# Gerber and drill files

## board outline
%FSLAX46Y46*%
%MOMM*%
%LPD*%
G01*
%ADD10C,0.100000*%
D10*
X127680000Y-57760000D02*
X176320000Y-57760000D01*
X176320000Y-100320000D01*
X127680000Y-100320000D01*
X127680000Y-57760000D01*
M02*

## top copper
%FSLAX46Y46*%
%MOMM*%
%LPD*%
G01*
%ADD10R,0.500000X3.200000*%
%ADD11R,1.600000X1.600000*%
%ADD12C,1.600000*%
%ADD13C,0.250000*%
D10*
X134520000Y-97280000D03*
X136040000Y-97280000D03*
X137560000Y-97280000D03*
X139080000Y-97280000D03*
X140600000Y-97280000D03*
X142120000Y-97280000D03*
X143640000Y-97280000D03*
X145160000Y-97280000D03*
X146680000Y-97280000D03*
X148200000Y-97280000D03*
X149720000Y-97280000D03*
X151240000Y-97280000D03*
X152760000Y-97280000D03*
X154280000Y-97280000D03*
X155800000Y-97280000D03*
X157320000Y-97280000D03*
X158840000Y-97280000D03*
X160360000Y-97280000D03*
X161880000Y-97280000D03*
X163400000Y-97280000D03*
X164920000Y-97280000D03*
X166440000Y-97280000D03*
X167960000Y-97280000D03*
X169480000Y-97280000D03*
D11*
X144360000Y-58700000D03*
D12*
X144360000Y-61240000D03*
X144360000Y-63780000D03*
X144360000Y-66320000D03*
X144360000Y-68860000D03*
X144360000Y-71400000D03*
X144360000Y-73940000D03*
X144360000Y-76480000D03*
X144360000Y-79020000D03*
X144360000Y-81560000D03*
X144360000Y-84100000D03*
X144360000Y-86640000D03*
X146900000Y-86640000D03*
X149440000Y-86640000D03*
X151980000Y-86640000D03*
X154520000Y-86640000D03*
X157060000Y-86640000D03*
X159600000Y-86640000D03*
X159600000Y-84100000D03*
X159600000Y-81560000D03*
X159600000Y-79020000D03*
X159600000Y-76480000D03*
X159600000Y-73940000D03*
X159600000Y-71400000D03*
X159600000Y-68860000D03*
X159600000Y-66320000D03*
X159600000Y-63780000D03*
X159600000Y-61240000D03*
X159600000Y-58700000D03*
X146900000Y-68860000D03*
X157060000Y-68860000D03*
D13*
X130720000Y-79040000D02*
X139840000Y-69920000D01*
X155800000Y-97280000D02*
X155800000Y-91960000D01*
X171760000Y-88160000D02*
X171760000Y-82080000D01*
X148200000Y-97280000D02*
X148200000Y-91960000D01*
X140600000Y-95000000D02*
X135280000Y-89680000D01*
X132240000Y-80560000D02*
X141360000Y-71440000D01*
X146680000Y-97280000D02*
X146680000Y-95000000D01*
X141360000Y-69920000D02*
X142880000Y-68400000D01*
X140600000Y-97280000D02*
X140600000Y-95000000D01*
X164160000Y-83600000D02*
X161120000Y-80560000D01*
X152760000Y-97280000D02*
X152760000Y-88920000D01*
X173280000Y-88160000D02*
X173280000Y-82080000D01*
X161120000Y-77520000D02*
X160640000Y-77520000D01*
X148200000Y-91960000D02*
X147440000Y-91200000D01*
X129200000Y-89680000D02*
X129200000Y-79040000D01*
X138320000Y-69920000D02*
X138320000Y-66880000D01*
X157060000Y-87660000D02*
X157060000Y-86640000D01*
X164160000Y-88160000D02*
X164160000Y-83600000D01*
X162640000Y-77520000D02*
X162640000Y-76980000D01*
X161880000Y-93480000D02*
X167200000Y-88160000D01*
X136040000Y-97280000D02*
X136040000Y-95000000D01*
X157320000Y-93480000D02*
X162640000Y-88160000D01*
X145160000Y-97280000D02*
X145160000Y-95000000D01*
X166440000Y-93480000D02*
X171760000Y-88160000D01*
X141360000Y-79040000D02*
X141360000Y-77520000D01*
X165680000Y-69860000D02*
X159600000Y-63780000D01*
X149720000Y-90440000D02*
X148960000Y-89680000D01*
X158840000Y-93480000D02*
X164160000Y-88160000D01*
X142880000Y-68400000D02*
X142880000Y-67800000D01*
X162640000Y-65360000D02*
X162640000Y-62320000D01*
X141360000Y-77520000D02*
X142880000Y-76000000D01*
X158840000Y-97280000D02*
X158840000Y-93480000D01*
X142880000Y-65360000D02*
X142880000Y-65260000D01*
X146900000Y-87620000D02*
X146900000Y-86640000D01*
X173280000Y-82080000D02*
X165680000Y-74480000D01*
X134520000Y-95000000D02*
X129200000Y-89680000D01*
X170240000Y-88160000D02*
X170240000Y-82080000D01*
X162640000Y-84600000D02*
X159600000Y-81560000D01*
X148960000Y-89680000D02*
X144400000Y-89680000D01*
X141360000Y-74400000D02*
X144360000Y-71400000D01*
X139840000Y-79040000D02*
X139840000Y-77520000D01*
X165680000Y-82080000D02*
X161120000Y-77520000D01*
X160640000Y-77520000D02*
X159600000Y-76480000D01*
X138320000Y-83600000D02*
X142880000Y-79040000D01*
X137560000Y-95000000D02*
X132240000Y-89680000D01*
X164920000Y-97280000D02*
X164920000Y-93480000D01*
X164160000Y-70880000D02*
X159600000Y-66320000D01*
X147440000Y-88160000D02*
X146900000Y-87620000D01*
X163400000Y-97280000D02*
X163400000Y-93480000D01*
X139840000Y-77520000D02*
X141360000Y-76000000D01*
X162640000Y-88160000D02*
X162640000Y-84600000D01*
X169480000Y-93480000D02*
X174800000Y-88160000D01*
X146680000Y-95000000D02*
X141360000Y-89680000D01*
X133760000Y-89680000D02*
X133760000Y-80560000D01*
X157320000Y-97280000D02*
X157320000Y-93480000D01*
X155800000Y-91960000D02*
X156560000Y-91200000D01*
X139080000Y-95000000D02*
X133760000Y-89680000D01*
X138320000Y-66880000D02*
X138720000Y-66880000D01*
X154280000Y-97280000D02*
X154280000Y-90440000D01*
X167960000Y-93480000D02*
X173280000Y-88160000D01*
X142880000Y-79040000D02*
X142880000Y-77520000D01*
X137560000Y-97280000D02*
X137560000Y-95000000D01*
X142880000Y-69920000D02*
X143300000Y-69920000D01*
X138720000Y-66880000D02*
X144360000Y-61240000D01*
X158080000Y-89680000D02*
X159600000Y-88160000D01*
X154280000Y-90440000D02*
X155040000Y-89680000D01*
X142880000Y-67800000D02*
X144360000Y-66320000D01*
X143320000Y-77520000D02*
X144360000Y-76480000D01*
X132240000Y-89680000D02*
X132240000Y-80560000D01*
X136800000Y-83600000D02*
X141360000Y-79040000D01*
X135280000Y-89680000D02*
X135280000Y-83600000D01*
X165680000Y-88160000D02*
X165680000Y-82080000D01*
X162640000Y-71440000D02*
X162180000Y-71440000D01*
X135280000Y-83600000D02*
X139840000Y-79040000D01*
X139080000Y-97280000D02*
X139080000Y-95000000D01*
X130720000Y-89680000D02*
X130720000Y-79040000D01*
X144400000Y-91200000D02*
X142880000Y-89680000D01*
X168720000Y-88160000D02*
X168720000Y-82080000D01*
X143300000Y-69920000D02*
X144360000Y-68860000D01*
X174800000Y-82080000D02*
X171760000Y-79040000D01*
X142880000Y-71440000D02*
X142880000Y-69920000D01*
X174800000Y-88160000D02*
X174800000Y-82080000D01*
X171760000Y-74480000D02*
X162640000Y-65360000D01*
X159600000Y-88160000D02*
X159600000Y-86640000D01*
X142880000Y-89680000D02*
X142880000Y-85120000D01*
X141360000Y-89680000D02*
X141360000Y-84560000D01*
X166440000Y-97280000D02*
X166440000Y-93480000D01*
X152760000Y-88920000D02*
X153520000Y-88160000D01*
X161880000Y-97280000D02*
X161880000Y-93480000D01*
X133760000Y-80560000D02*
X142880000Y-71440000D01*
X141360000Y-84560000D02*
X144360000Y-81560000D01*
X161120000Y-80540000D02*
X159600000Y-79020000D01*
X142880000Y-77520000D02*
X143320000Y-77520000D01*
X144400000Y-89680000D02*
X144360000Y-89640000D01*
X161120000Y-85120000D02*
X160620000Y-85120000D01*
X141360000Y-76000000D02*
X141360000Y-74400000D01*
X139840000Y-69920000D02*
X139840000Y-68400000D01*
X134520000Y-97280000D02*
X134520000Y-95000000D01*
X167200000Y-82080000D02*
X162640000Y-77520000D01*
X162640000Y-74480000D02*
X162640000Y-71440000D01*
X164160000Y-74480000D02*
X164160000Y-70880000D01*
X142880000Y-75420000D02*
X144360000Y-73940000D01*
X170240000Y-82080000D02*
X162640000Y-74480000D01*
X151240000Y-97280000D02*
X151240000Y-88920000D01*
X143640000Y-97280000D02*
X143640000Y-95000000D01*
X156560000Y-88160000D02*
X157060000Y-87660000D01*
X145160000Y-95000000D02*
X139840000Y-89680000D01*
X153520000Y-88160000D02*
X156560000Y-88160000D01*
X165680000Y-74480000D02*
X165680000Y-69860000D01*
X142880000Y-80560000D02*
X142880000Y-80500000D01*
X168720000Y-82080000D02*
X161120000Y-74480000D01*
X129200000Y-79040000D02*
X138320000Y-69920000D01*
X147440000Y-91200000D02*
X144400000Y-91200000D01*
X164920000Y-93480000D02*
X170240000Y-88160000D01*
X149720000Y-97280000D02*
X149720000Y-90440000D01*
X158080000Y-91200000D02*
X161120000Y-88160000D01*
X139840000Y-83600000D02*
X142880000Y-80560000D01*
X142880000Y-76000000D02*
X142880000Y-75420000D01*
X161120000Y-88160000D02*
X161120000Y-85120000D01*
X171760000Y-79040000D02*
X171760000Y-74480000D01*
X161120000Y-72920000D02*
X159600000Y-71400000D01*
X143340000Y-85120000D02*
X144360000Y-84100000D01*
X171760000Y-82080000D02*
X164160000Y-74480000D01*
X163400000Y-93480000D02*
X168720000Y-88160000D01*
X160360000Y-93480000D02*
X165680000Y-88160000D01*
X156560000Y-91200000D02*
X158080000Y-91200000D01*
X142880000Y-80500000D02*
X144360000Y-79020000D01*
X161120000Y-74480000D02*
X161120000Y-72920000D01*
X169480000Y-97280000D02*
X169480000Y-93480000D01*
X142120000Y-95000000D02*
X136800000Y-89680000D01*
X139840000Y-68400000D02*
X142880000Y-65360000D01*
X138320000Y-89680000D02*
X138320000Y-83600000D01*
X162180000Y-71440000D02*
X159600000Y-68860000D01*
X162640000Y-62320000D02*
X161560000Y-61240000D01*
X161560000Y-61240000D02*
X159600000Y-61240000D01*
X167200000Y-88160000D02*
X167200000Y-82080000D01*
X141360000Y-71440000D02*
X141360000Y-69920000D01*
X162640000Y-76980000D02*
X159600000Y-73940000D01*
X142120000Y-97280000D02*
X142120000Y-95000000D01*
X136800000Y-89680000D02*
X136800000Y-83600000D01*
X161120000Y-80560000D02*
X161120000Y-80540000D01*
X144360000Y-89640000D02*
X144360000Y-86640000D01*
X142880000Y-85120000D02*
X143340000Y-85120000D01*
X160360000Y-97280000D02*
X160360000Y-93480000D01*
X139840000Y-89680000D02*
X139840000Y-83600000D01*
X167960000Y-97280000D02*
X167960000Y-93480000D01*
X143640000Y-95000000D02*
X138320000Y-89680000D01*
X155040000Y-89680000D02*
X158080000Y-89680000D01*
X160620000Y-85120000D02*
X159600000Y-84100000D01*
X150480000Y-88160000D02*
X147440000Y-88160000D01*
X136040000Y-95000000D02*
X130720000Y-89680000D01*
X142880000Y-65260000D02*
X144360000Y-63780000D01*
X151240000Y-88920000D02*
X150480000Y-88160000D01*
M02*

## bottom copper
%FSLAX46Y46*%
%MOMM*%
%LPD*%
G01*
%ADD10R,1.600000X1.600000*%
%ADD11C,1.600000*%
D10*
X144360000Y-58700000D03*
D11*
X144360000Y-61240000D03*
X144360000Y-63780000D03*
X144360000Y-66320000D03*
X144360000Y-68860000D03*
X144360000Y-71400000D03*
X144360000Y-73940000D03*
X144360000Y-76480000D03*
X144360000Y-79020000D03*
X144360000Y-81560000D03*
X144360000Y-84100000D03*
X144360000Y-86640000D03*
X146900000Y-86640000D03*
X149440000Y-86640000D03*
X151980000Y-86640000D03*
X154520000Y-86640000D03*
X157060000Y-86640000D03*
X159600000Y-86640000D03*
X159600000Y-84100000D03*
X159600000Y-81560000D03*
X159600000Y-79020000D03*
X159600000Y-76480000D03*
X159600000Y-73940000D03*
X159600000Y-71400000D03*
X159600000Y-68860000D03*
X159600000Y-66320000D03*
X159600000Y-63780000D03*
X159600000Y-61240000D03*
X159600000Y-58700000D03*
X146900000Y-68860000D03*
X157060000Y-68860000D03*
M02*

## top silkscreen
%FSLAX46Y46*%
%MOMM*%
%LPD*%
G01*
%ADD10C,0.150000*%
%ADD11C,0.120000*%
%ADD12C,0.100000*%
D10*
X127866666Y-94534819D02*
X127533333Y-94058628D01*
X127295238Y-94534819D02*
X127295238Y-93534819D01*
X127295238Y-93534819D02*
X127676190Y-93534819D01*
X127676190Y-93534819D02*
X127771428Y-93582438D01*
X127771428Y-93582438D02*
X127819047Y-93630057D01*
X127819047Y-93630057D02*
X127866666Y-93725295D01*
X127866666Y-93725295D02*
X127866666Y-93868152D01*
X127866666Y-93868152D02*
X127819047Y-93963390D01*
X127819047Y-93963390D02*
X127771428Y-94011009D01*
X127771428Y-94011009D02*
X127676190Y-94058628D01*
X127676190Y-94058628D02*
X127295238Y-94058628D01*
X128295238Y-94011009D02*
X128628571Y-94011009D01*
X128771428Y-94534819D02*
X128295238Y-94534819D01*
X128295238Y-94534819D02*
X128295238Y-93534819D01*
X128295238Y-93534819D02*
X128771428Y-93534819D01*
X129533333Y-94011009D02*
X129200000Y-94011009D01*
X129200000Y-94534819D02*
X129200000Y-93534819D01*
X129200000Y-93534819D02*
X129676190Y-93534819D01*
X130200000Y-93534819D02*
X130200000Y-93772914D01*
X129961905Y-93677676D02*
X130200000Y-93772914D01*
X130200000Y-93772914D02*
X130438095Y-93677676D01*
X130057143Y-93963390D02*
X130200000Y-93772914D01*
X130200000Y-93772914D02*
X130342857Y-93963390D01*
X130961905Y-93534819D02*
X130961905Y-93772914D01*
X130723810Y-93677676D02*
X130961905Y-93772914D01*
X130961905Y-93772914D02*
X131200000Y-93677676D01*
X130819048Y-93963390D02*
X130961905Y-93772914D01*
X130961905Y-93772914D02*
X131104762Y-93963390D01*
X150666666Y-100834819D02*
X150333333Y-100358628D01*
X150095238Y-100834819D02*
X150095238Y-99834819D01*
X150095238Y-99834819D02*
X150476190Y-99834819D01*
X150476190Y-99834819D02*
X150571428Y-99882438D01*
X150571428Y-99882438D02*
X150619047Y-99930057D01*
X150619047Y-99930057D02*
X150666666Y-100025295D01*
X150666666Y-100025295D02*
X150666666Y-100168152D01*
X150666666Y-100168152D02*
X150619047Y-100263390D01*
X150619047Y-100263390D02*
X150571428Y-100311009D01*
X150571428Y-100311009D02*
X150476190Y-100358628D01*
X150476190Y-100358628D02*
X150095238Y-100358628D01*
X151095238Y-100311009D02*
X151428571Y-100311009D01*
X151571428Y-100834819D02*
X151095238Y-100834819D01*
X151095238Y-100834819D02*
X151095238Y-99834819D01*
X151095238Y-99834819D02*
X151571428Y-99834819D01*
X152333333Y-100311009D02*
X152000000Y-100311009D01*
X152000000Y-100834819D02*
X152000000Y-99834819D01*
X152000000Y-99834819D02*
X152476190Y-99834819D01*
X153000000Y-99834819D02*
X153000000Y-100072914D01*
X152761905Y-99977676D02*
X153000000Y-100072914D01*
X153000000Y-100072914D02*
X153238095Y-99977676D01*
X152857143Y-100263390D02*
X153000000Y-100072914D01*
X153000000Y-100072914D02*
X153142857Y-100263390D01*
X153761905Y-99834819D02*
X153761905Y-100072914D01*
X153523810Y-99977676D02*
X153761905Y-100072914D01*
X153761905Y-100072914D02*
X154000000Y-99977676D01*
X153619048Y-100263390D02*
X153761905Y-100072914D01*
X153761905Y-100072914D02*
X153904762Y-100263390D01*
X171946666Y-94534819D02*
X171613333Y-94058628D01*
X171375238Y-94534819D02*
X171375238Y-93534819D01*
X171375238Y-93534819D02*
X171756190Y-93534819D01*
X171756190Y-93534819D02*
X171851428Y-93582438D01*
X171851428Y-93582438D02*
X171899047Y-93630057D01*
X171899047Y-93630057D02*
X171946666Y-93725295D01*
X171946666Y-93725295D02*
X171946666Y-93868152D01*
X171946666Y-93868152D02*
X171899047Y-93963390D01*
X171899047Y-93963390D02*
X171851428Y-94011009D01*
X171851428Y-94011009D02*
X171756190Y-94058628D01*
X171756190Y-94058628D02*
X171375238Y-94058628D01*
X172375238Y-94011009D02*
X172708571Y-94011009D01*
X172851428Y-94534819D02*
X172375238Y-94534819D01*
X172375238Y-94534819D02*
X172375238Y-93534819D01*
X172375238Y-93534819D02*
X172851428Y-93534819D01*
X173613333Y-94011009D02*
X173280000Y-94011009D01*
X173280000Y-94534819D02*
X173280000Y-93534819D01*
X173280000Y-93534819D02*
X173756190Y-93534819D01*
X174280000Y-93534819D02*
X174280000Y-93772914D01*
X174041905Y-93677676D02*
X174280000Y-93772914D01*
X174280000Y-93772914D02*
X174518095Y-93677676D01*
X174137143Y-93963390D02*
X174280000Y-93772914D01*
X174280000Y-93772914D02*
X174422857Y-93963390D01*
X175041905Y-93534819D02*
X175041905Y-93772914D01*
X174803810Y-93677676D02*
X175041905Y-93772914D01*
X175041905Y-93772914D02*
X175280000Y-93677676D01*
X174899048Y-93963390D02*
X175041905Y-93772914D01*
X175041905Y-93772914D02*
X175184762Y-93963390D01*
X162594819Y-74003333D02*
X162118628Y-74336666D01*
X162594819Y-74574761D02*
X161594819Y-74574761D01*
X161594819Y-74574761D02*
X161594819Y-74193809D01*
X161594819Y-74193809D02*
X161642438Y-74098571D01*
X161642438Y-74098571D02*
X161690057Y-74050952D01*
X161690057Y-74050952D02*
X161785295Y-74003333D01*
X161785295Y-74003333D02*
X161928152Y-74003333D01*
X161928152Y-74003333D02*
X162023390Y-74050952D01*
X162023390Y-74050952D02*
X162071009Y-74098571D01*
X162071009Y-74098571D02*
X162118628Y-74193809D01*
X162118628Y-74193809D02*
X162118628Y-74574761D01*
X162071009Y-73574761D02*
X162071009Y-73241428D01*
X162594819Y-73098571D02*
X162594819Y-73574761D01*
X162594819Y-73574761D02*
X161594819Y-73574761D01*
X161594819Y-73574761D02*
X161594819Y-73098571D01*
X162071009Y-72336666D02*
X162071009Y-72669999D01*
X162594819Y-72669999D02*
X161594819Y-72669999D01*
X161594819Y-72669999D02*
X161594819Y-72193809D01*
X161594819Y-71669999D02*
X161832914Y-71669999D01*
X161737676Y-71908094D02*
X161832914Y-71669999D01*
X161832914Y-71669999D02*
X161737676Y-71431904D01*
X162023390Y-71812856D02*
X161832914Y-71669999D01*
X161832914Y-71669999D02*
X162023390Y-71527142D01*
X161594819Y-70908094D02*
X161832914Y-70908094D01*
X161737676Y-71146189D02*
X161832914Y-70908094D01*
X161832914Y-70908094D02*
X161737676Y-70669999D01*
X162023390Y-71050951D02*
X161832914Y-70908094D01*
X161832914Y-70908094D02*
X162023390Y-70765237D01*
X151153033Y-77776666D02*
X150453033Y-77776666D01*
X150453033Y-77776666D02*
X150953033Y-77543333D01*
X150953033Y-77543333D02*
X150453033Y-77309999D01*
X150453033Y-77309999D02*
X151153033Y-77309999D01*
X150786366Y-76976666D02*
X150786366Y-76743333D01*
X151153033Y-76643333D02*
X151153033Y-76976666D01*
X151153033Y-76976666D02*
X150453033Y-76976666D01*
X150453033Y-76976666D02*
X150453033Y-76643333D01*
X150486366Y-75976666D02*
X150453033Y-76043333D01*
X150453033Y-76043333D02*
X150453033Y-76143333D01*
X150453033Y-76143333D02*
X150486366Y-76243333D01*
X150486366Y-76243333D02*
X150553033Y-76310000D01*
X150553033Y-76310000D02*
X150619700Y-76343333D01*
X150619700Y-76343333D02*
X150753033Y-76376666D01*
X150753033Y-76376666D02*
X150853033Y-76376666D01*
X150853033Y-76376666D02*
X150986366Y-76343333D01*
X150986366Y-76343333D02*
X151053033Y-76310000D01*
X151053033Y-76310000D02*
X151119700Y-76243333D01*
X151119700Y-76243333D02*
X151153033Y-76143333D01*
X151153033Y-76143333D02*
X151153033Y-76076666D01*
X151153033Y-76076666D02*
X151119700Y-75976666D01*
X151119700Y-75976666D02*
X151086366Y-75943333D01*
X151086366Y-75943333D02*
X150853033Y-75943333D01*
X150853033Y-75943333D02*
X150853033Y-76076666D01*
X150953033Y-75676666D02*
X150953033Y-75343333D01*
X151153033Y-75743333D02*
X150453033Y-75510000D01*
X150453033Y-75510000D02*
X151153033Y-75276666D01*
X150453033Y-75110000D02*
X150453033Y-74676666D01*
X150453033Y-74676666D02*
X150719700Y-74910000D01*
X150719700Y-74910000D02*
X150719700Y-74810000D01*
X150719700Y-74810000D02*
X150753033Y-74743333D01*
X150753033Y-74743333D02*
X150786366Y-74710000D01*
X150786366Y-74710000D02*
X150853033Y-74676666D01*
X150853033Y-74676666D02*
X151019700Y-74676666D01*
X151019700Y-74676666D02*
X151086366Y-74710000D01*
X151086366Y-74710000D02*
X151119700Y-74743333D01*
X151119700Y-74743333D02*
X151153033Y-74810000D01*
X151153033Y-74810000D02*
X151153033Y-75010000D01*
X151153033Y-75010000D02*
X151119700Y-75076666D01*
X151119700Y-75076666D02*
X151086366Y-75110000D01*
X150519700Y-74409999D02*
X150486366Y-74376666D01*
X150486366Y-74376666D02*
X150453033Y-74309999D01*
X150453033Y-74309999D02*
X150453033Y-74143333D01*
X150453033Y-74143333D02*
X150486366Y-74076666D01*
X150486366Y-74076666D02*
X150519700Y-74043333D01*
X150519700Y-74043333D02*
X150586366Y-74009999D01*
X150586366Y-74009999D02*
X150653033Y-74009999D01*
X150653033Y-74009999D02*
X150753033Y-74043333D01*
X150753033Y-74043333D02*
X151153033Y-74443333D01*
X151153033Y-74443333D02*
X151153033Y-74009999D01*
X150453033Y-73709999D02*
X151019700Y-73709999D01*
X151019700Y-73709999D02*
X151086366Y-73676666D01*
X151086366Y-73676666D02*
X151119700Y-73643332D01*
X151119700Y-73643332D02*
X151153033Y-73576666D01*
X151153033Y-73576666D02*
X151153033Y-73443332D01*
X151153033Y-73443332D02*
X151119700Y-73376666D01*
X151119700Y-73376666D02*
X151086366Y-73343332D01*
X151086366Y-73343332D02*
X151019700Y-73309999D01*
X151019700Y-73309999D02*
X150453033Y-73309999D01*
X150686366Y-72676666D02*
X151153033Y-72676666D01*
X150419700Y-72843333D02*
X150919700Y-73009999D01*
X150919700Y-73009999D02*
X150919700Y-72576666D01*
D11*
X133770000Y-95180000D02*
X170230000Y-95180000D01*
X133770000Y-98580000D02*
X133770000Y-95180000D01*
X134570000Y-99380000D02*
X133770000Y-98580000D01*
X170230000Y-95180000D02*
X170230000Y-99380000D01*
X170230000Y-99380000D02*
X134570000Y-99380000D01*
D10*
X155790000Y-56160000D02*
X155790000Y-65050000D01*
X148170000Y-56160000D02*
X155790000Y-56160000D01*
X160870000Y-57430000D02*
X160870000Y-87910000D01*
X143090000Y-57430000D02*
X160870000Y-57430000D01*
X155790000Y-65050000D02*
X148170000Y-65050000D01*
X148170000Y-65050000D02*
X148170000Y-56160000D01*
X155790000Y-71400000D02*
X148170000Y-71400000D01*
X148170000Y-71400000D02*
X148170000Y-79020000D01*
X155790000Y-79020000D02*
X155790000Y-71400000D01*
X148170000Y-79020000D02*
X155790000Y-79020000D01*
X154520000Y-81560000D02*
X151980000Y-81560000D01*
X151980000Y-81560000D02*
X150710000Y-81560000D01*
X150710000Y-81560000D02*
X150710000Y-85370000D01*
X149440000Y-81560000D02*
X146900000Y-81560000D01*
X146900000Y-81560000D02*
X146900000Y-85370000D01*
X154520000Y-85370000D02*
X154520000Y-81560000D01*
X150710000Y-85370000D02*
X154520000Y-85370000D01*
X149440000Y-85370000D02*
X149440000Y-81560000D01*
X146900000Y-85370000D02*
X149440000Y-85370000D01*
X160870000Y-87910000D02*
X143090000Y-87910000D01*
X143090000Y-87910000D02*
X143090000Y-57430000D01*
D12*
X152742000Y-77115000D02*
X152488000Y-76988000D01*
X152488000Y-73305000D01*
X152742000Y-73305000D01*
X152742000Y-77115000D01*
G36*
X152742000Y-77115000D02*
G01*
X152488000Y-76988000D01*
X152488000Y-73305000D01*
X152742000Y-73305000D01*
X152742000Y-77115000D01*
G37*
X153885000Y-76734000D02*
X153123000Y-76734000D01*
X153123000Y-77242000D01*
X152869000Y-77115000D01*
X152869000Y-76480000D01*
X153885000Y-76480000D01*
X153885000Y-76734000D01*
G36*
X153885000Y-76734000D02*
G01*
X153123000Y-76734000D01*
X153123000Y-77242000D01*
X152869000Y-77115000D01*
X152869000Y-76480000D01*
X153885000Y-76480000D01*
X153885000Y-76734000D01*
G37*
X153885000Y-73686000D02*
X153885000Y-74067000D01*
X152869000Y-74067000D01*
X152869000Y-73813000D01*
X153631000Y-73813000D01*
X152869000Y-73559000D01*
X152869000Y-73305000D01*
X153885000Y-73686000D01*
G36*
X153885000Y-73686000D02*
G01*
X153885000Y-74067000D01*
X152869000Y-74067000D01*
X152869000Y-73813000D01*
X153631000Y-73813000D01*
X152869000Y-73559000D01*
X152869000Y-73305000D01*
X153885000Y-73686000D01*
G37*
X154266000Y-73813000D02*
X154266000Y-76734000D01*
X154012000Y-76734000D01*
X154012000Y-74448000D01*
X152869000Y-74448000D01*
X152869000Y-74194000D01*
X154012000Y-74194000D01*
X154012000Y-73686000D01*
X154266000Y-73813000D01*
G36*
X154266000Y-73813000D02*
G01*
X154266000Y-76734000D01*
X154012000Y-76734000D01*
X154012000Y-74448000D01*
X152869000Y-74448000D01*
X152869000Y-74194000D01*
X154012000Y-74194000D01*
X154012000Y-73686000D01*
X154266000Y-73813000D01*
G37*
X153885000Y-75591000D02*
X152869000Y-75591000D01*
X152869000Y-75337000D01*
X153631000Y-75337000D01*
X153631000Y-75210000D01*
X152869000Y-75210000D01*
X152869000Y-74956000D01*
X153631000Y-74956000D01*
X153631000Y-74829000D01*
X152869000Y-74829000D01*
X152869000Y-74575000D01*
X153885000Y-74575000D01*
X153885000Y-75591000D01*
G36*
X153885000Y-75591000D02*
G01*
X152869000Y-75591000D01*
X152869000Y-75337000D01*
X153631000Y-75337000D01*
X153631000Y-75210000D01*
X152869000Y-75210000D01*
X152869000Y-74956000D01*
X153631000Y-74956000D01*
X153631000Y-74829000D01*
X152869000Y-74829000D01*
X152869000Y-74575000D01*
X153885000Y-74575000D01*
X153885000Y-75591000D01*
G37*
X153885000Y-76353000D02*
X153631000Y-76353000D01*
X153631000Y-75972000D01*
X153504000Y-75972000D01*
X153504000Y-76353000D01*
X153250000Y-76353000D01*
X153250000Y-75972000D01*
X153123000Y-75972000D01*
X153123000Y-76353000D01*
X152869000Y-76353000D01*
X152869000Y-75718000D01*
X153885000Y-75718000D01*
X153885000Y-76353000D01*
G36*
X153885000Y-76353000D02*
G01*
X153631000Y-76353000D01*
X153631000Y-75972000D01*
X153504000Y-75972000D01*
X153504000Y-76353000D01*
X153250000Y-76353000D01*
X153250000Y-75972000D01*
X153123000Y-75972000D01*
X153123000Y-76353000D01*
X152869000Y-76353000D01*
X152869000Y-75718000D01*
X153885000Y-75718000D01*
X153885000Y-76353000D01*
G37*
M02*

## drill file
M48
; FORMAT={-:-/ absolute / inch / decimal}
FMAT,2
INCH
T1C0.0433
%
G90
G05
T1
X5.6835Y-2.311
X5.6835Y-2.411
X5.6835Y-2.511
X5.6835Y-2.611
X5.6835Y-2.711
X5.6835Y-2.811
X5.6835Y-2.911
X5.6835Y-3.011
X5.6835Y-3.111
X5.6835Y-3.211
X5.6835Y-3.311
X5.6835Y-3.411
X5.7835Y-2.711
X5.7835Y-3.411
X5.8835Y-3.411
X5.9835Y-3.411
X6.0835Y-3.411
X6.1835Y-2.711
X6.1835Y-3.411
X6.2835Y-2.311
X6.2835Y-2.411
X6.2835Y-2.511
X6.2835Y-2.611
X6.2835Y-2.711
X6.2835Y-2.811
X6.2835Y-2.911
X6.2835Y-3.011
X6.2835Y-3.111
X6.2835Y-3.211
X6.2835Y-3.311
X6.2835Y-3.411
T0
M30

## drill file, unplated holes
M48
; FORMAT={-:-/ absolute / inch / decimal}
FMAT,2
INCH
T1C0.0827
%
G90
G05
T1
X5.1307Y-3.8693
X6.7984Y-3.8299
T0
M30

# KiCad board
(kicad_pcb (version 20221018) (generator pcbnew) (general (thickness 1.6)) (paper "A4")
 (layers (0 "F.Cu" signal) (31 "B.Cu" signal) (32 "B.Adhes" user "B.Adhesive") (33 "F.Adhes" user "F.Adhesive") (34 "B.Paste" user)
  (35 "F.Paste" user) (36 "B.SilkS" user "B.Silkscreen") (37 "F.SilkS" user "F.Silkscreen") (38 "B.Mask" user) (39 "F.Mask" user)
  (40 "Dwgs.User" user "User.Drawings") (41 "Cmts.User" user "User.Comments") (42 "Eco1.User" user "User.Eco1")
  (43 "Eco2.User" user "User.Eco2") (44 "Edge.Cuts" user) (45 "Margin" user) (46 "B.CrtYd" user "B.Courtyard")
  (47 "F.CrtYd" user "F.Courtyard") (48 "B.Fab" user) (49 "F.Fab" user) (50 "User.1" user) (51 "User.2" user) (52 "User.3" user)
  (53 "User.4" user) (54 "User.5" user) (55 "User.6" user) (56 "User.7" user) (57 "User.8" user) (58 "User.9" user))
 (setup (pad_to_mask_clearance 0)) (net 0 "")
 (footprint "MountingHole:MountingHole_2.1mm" (layer "F.Cu") (at 129.2 97.28)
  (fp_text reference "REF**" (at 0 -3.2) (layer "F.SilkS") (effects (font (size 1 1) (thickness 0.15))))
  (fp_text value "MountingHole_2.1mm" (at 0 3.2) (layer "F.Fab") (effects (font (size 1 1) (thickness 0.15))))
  (pad "" np_thru_hole circle (at 1.12 1) (size 2.1 2.1) (drill 2.1) (layers "F&B.Cu" "*.Mask")))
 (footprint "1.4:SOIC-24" (layer "F.Cu") (at 152 97.28)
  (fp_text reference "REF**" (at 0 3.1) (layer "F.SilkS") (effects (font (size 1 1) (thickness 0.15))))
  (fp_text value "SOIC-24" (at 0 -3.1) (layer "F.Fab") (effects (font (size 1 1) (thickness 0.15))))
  (fp_line (start -18.23 -2.1) (end 18.23 -2.1) (stroke (width 0.12) (type default)) (layer "F.SilkS"))
  (fp_line (start -18.23 1.3) (end -18.23 -2.1) (stroke (width 0.12) (type default)) (layer "F.SilkS"))
  (fp_line (start -17.43 2.1) (end -18.23 1.3) (stroke (width 0.12) (type default)) (layer "F.SilkS"))
  (fp_line (start 18.23 -2.1) (end 18.23 2.1) (stroke (width 0.12) (type default)) (layer "F.SilkS"))
  (fp_line (start 18.23 2.1) (end -17.43 2.1) (stroke (width 0.12) (type default)) (layer "F.SilkS"))
  (pad "1" smd rect (at -17.48 0) (size 0.5 3.2) (layers "F.Cu" "F.Paste" "F.Mask") (thermal_bridge_angle 45))
  (pad "2" smd rect (at -15.96 0) (size 0.5 3.2) (layers "F.Cu" "F.Paste" "F.Mask") (thermal_bridge_angle 45))
  (pad "3" smd rect (at -14.44 0) (size 0.5 3.2) (layers "F.Cu" "F.Paste" "F.Mask") (thermal_bridge_angle 45))
  (pad "4" smd rect (at -12.92 0) (size 0.5 3.2) (layers "F.Cu" "F.Paste" "F.Mask") (thermal_bridge_angle 45))
  (pad "5" smd rect (at -11.4 0) (size 0.5 3.2) (layers "F.Cu" "F.Paste" "F.Mask") (thermal_bridge_angle 45))
  (pad "6" smd rect (at -9.88 0) (size 0.5 3.2) (layers "F.Cu" "F.Paste" "F.Mask") (thermal_bridge_angle 45))
  (pad "7" smd rect (at -8.36 0) (size 0.5 3.2) (layers "F.Cu" "F.Paste" "F.Mask") (thermal_bridge_angle 45))
  (pad "8" smd rect (at -6.84 0) (size 0.5 3.2) (layers "F.Cu" "F.Paste" "F.Mask") (thermal_bridge_angle 45))
  (pad "9" smd rect (at -5.32 0) (size 0.5 3.2) (layers "F.Cu" "F.Paste" "F.Mask") (thermal_bridge_angle 45))
  (pad "10" smd rect (at -3.8 0) (size 0.5 3.2) (layers "F.Cu" "F.Paste" "F.Mask") (thermal_bridge_angle 45))
  (pad "11" smd rect (at -2.28 0) (size 0.5 3.2) (layers "F.Cu" "F.Paste" "F.Mask") (thermal_bridge_angle 45))
  (pad "12" smd rect (at -0.76 0) (size 0.5 3.2) (layers "F.Cu" "F.Paste" "F.Mask") (thermal_bridge_angle 45))
  (pad "13" smd rect (at 0.76 0) (size 0.5 3.2) (layers "F.Cu" "F.Paste" "F.Mask") (thermal_bridge_angle 45))
  (pad "14" smd rect (at 2.28 0) (size 0.5 3.2) (layers "F.Cu" "F.Paste" "F.Mask") (thermal_bridge_angle 45))
  (pad "15" smd rect (at 3.8 0) (size 0.5 3.2) (layers "F.Cu" "F.Paste" "F.Mask") (thermal_bridge_angle 45))
  (pad "16" smd rect (at 5.32 0) (size 0.5 3.2) (layers "F.Cu" "F.Paste" "F.Mask") (thermal_bridge_angle 45))
  (pad "17" smd rect (at 6.84 0) (size 0.5 3.2) (layers "F.Cu" "F.Paste" "F.Mask") (thermal_bridge_angle 45))
  (pad "18" smd rect (at 8.36 0) (size 0.5 3.2) (layers "F.Cu" "F.Paste" "F.Mask") (thermal_bridge_angle 45))
  (pad "19" smd rect (at 9.88 0) (size 0.5 3.2) (layers "F.Cu" "F.Paste" "F.Mask") (thermal_bridge_angle 45))
  (pad "20" smd rect (at 11.4 0) (size 0.5 3.2) (layers "F.Cu" "F.Paste" "F.Mask") (thermal_bridge_angle 45))
  (pad "21" smd rect (at 12.92 0) (size 0.5 3.2) (layers "F.Cu" "F.Paste" "F.Mask") (thermal_bridge_angle 45))
  (pad "22" smd rect (at 14.44 0) (size 0.5 3.2) (layers "F.Cu" "F.Paste" "F.Mask") (thermal_bridge_angle 45))
  (pad "23" smd rect (at 15.96 0) (size 0.5 3.2) (layers "F.Cu" "F.Paste" "F.Mask") (thermal_bridge_angle 45))
  (pad "24" smd rect (at 17.48 0) (size 0.5 3.2) (layers "F.Cu" "F.Paste" "F.Mask") (thermal_bridge_angle 45)))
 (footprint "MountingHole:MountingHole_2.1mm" (layer "F.Cu") (at 173.28 97.28)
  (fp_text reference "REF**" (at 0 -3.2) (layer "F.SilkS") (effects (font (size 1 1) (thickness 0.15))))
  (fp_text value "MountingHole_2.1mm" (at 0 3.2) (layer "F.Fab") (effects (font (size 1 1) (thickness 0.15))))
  (pad "" np_thru_hole circle (at -0.6 0) (size 2.1 2.1) (drill 2.1) (layers "F&B.Cu" "*.Mask")))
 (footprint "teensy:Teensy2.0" (layer "F.Cu") (at 151.98 72.67 -90)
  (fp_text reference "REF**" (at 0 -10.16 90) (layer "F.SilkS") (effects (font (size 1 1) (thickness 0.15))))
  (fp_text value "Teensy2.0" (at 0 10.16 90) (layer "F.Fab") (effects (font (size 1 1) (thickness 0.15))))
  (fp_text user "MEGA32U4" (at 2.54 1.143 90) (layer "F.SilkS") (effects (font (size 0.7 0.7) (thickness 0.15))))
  (fp_line (start -16.51 -3.81) (end -7.62 -3.81) (stroke (width 0.15) (type solid)) (layer "F.SilkS"))
  (fp_line (start -16.51 3.81) (end -16.51 -3.81) (stroke (width 0.15) (type solid)) (layer "F.SilkS"))
  (fp_line (start -15.24 -8.89) (end 15.24 -8.89) (stroke (width 0.15) (type solid)) (layer "F.SilkS"))
  (fp_line (start -15.24 8.89) (end -15.24 -8.89) (stroke (width 0.15) (type solid)) (layer "F.SilkS"))
  (fp_line (start -7.62 -3.81) (end -7.62 3.81) (stroke (width 0.15) (type solid)) (layer "F.SilkS"))
  (fp_line (start -7.62 3.81) (end -16.51 3.81) (stroke (width 0.15) (type solid)) (layer "F.SilkS"))
  (fp_line (start -1.27 -3.81) (end -1.27 3.81) (stroke (width 0.15) (type solid)) (layer "F.SilkS"))
  (fp_line (start -1.27 3.81) (end 6.35 3.81) (stroke (width 0.15) (type solid)) (layer "F.SilkS"))
  (fp_line (start 6.35 -3.81) (end -1.27 -3.81) (stroke (width 0.15) (type solid)) (layer "F.SilkS"))
  (fp_line (start 6.35 3.81) (end 6.35 -3.81) (stroke (width 0.15) (type solid)) (layer "F.SilkS"))
  (fp_line (start 8.89 -2.54) (end 8.89 0) (stroke (width 0.15) (type solid)) (layer "F.SilkS"))
  (fp_line (start 8.89 0) (end 8.89 1.27) (stroke (width 0.15) (type solid)) (layer "F.SilkS"))
  (fp_line (start 8.89 1.27) (end 12.7 1.27) (stroke (width 0.15) (type solid)) (layer "F.SilkS"))
  (fp_line (start 8.89 2.54) (end 8.89 5.08) (stroke (width 0.15) (type solid)) (layer "F.SilkS"))
  (fp_line (start 8.89 5.08) (end 12.7 5.08) (stroke (width 0.15) (type solid)) (layer "F.SilkS"))
  (fp_line (start 12.7 -2.54) (end 8.89 -2.54) (stroke (width 0.15) (type solid)) (layer "F.SilkS"))
  (fp_line (start 12.7 1.27) (end 12.7 -2.54) (stroke (width 0.15) (type solid)) (layer "F.SilkS"))
  (fp_line (start 12.7 2.54) (end 8.89 2.54) (stroke (width 0.15) (type solid)) (layer "F.SilkS"))
  (fp_line (start 12.7 5.08) (end 12.7 2.54) (stroke (width 0.15) (type solid)) (layer "F.SilkS"))
  (fp_line (start 15.24 -8.89) (end 15.24 8.89) (stroke (width 0.15) (type solid)) (layer "F.SilkS"))
  (fp_line (start 15.24 8.89) (end -15.24 8.89) (stroke (width 0.15) (type solid)) (layer "F.SilkS"))
  (fp_poly
   (pts (xy 0.635 -0.762) (xy 4.445 -0.762) (xy 4.318 -0.508) (xy 0.635 -0.508)) (stroke (width 0.1) (type solid)) (fill solid)
   (layer "F.SilkS"))
  (fp_poly
   (pts (xy 3.81 -1.905) (xy 3.81 -0.889) (xy 4.445 -0.889) (xy 4.572 -1.143) (xy 4.064 -1.143) (xy 4.064 -1.905))
   (stroke (width 0.1) (type solid)) (fill solid) (layer "F.SilkS"))
  (fp_poly
   (pts (xy 1.397 -0.889) (xy 1.397 -1.905) (xy 1.016 -1.905) (xy 0.635 -0.889) (xy 0.889 -0.889) (xy 1.143 -1.651) (xy 1.143 -0.889))
   (stroke (width 0.1) (type solid)) (fill solid) (layer "F.SilkS"))
  (fp_poly
   (pts (xy 4.064 -2.032) (xy 1.778 -2.032) (xy 1.778 -0.889) (xy 1.524 -0.889) (xy 1.524 -2.032) (xy 1.016 -2.032) (xy 1.143 -2.286)
    (xy 4.064 -2.286))
   (stroke (width 0.1) (type solid)) (fill solid) (layer "F.SilkS"))
  (fp_poly
   (pts (xy 2.921 -0.889) (xy 2.921 -1.905) (xy 1.905 -1.905) (xy 1.905 -0.889) (xy 2.159 -0.889) (xy 2.159 -1.651) (xy 2.286 -1.651)
    (xy 2.286 -0.889) (xy 2.54 -0.889) (xy 2.54 -1.651) (xy 2.667 -1.651) (xy 2.667 -0.889))
   (stroke (width 0.1) (type solid)) (fill solid) (layer "F.SilkS"))
  (fp_poly
   (pts (xy 3.048 -1.905) (xy 3.683 -1.905) (xy 3.683 -1.651) (xy 3.302 -1.651) (xy 3.302 -1.524) (xy 3.683 -1.524) (xy 3.683 -1.27)
    (xy 3.302 -1.27) (xy 3.302 -1.143) (xy 3.683 -1.143) (xy 3.683 -0.889) (xy 3.048 -0.889))
   (stroke (width 0.1) (type solid)) (fill solid) (layer "F.SilkS"))
  (pad "1" thru_hole rect (at -13.97 7.62 270) (size 1.6 1.6) (drill 1.1) (layers "*.Cu" "*.Mask"))
  (pad "2" thru_hole circle (at -11.43 7.62 270) (size 1.6 1.6) (drill 1.1) (layers "*.Cu" "*.Mask"))
  (pad "3" thru_hole circle (at -8.89 7.62 270) (size 1.6 1.6) (drill 1.1) (layers "*.Cu" "*.Mask"))
  (pad "4" thru_hole circle (at -6.35 7.62 270) (size 1.6 1.6) (drill 1.1) (layers "*.Cu" "*.Mask"))
  (pad "5" thru_hole circle (at -3.81 7.62 270) (size 1.6 1.6) (drill 1.1) (layers "*.Cu" "*.Mask"))
  (pad "6" thru_hole circle (at -1.27 7.62 270) (size 1.6 1.6) (drill 1.1) (layers "*.Cu" "*.Mask"))
  (pad "7" thru_hole circle (at 1.27 7.62 270) (size 1.6 1.6) (drill 1.1) (layers "*.Cu" "*.Mask"))
  (pad "8" thru_hole circle (at 3.81 7.62 270) (size 1.6 1.6) (drill 1.1) (layers "*.Cu" "*.Mask"))
  (pad "9" thru_hole circle (at 6.35 7.62 270) (size 1.6 1.6) (drill 1.1) (layers "*.Cu" "*.Mask"))
  (pad "10" thru_hole circle (at 8.89 7.62 270) (size 1.6 1.6) (drill 1.1) (layers "*.Cu" "*.Mask"))
  (pad "11" thru_hole circle (at 11.43 7.62 270) (size 1.6 1.6) (drill 1.1) (layers "*.Cu" "*.Mask"))
  (pad "12" thru_hole circle (at 13.97 7.62 270) (size 1.6 1.6) (drill 1.1) (layers "*.Cu" "*.Mask"))
  (pad "13" thru_hole circle (at 13.97 5.08 270) (size 1.6 1.6) (drill 1.1) (layers "*.Cu" "*.Mask"))
  (pad "14" thru_hole circle (at 13.97 2.54 270) (size 1.6 1.6) (drill 1.1) (layers "*.Cu" "*.Mask"))
  (pad "15" thru_hole circle (at 13.97 0 270) (size 1.6 1.6) (drill 1.1) (layers "*.Cu" "*.Mask"))
  (pad "16" thru_hole circle (at 13.97 -2.54 270) (size 1.6 1.6) (drill 1.1) (layers "*.Cu" "*.Mask"))
  (pad "17" thru_hole circle (at 13.97 -5.08 270) (size 1.6 1.6) (drill 1.1) (layers "*.Cu" "*.Mask"))
  (pad "18" thru_hole circle (at 13.97 -7.62 270) (size 1.6 1.6) (drill 1.1) (layers "*.Cu" "*.Mask"))
  (pad "19" thru_hole circle (at 11.43 -7.62 270) (size 1.6 1.6) (drill 1.1) (layers "*.Cu" "*.Mask"))
  (pad "20" thru_hole circle (at 8.89 -7.62 270) (size 1.6 1.6) (drill 1.1) (layers "*.Cu" "*.Mask"))
  (pad "21" thru_hole circle (at 6.35 -7.62 270) (size 1.6 1.6) (drill 1.1) (layers "*.Cu" "*.Mask"))
  (pad "22" thru_hole circle (at 3.81 -7.62 270) (size 1.6 1.6) (drill 1.1) (layers "*.Cu" "*.Mask"))
  (pad "23" thru_hole circle (at 1.27 -7.62 270) (size 1.6 1.6) (drill 1.1) (layers "*.Cu" "*.Mask"))
  (pad "24" thru_hole circle (at -1.27 -7.62 270) (size 1.6 1.6) (drill 1.1) (layers "*.Cu" "*.Mask"))
  (pad "25" thru_hole circle (at -3.81 -7.62 270) (size 1.6 1.6) (drill 1.1) (layers "*.Cu" "*.Mask"))
  (pad "26" thru_hole circle (at -6.35 -7.62 270) (size 1.6 1.6) (drill 1.1) (layers "*.Cu" "*.Mask"))
  (pad "27" thru_hole circle (at -8.89 -7.62 270) (size 1.6 1.6) (drill 1.1) (layers "*.Cu" "*.Mask"))
  (pad "28" thru_hole circle (at -11.43 -7.62 270) (size 1.6 1.6) (drill 1.1) (layers "*.Cu" "*.Mask"))
  (pad "29" thru_hole circle (at -13.97 -7.62 270) (size 1.6 1.6) (drill 1.1) (layers "*.Cu" "*.Mask"))
  (pad "30" thru_hole circle (at -3.81 5.08 270) (size 1.6 1.6) (drill 1.1) (layers "*.Cu" "*.Mask"))
  (pad "31" thru_hole circle (at -3.81 -5.08 270) (size 1.6 1.6) (drill 1.1) (layers "*.Cu" "*.Mask")))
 (gr_rect (start 127.68 57.76) (end 176.32 100.32) (stroke (width 0.1) (type default)) (fill none) (layer "Edge.Cuts"))
 (segment (start 130.72 79.04) (end 139.84 69.92) (width 0.25) (layer "F.Cu") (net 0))
 (segment (start 155.8 97.28) (end 155.8 91.96) (width 0.25) (layer "F.Cu") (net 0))
 (segment (start 171.76 88.16) (end 171.76 82.08) (width 0.25) (layer "F.Cu") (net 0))
 (segment (start 148.2 97.28) (end 148.2 91.96) (width 0.25) (layer "F.Cu") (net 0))
 (segment (start 140.6 95) (end 135.28 89.68) (width 0.25) (layer "F.Cu") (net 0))
 (segment (start 132.24 80.56) (end 141.36 71.44) (width 0.25) (layer "F.Cu") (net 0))
 (segment (start 146.68 97.28) (end 146.68 95) (width 0.25) (layer "F.Cu") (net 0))
 (segment (start 141.36 69.92) (end 142.88 68.4) (width 0.25) (layer "F.Cu") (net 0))
 (segment (start 140.6 97.28) (end 140.6 95) (width 0.25) (layer "F.Cu") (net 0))
 (segment (start 164.16 83.6) (end 161.12 80.56) (width 0.25) (layer "F.Cu") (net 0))
 (segment (start 152.76 97.28) (end 152.76 88.92) (width 0.25) (layer "F.Cu") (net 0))
 (segment (start 173.28 88.16) (end 173.28 82.08) (width 0.25) (layer "F.Cu") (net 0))
 (segment (start 161.12 77.52) (end 160.64 77.52) (width 0.25) (layer "F.Cu") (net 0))
 (segment (start 148.2 91.96) (end 147.44 91.2) (width 0.25) (layer "F.Cu") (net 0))
 (segment (start 129.2 89.68) (end 129.2 79.04) (width 0.25) (layer "F.Cu") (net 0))
 (segment (start 138.32 69.92) (end 138.32 66.88) (width 0.25) (layer "F.Cu") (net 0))
 (segment (start 157.06 87.66) (end 157.06 86.64) (width 0.25) (layer "F.Cu") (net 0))
 (segment (start 164.16 88.16) (end 164.16 83.6) (width 0.25) (layer "F.Cu") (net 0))
 (segment (start 162.64 77.52) (end 162.64 76.98) (width 0.25) (layer "F.Cu") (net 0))
 (segment (start 161.88 93.48) (end 167.2 88.16) (width 0.25) (layer "F.Cu") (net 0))
 (segment (start 136.04 97.28) (end 136.04 95) (width 0.25) (layer "F.Cu") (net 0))
 (segment (start 157.32 93.48) (end 162.64 88.16) (width 0.25) (layer "F.Cu") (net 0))
 (segment (start 145.16 97.28) (end 145.16 95) (width 0.25) (layer "F.Cu") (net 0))
 (segment (start 166.44 93.48) (end 171.76 88.16) (width 0.25) (layer "F.Cu") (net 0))
 (segment (start 141.36 79.04) (end 141.36 77.52) (width 0.25) (layer "F.Cu") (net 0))
 (segment (start 165.68 69.86) (end 159.6 63.78) (width 0.25) (layer "F.Cu") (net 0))
 (segment (start 149.72 90.44) (end 148.96 89.68) (width 0.25) (layer "F.Cu") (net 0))
 (segment (start 158.84 93.48) (end 164.16 88.16) (width 0.25) (layer "F.Cu") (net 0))
 (segment (start 142.88 68.4) (end 142.88 67.8) (width 0.25) (layer "F.Cu") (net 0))
 (segment (start 162.64 65.36) (end 162.64 62.32) (width 0.25) (layer "F.Cu") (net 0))
 (segment (start 141.36 77.52) (end 142.88 76) (width 0.25) (layer "F.Cu") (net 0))
 (segment (start 158.84 97.28) (end 158.84 93.48) (width 0.25) (layer "F.Cu") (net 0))
 (segment (start 142.88 65.36) (end 142.88 65.26) (width 0.25) (layer "F.Cu") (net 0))
 (segment (start 146.9 87.62) (end 146.9 86.64) (width 0.25) (layer "F.Cu") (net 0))
 (segment (start 173.28 82.08) (end 165.68 74.48) (width 0.25) (layer "F.Cu") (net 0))
 (segment (start 134.52 95) (end 129.2 89.68) (width 0.25) (layer "F.Cu") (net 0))
 (segment (start 170.24 88.16) (end 170.24 82.08) (width 0.25) (layer "F.Cu") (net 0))
 (segment (start 162.64 84.6) (end 159.6 81.56) (width 0.25) (layer "F.Cu") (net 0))
 (segment (start 148.96 89.68) (end 144.4 89.68) (width 0.25) (layer "F.Cu") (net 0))
 (segment (start 141.36 74.4) (end 144.36 71.4) (width 0.25) (layer "F.Cu") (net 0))
 (segment (start 139.84 79.04) (end 139.84 77.52) (width 0.25) (layer "F.Cu") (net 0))
 (segment (start 165.68 82.08) (end 161.12 77.52) (width 0.25) (layer "F.Cu") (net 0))
 (segment (start 160.64 77.52) (end 159.6 76.48) (width 0.25) (layer "F.Cu") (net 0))
 (segment (start 138.32 83.6) (end 142.88 79.04) (width 0.25) (layer "F.Cu") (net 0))
 (segment (start 137.56 95) (end 132.24 89.68) (width 0.25) (layer "F.Cu") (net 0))
 (segment (start 164.92 97.28) (end 164.92 93.48) (width 0.25) (layer "F.Cu") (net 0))
 (segment (start 164.16 70.88) (end 159.6 66.32) (width 0.25) (layer "F.Cu") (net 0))
 (segment (start 147.44 88.16) (end 146.9 87.62) (width 0.25) (layer "F.Cu") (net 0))
 (segment (start 163.4 97.28) (end 163.4 93.48) (width 0.25) (layer "F.Cu") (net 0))
 (segment (start 139.84 77.52) (end 141.36 76) (width 0.25) (layer "F.Cu") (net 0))
 (segment (start 162.64 88.16) (end 162.64 84.6) (width 0.25) (layer "F.Cu") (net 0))
 (segment (start 169.48 93.48) (end 174.8 88.16) (width 0.25) (layer "F.Cu") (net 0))
 (segment (start 146.68 95) (end 141.36 89.68) (width 0.25) (layer "F.Cu") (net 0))
 (segment (start 133.76 89.68) (end 133.76 80.56) (width 0.25) (layer "F.Cu") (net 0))
 (segment (start 157.32 97.28) (end 157.32 93.48) (width 0.25) (layer "F.Cu") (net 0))
 (segment (start 155.8 91.96) (end 156.56 91.2) (width 0.25) (layer "F.Cu") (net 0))
 (segment (start 139.08 95) (end 133.76 89.68) (width 0.25) (layer "F.Cu") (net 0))
 (segment (start 138.32 66.88) (end 138.72 66.88) (width 0.25) (layer "F.Cu") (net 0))
 (segment (start 154.28 97.28) (end 154.28 90.44) (width 0.25) (layer "F.Cu") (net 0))
 (segment (start 167.96 93.48) (end 173.28 88.16) (width 0.25) (layer "F.Cu") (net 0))
 (segment (start 142.88 79.04) (end 142.88 77.52) (width 0.25) (layer "F.Cu") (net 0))
 (segment (start 137.56 97.28) (end 137.56 95) (width 0.25) (layer "F.Cu") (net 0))
 (segment (start 142.88 69.92) (end 143.3 69.92) (width 0.25) (layer "F.Cu") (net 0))
 (segment (start 138.72 66.88) (end 144.36 61.24) (width 0.25) (layer "F.Cu") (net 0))
 (segment (start 158.08 89.68) (end 159.6 88.16) (width 0.25) (layer "F.Cu") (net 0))
 (segment (start 154.28 90.44) (end 155.04 89.68) (width 0.25) (layer "F.Cu") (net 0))
 (segment (start 142.88 67.8) (end 144.36 66.32) (width 0.25) (layer "F.Cu") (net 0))
 (segment (start 143.32 77.52) (end 144.36 76.48) (width 0.25) (layer "F.Cu") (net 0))
 (segment (start 132.24 89.68) (end 132.24 80.56) (width 0.25) (layer "F.Cu") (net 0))
 (segment (start 136.8 83.6) (end 141.36 79.04) (width 0.25) (layer "F.Cu") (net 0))
 (segment (start 135.28 89.68) (end 135.28 83.6) (width 0.25) (layer "F.Cu") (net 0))
 (segment (start 165.68 88.16) (end 165.68 82.08) (width 0.25) (layer "F.Cu") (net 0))
 (segment (start 162.64 71.44) (end 162.18 71.44) (width 0.25) (layer "F.Cu") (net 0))
 (segment (start 135.28 83.6) (end 139.84 79.04) (width 0.25) (layer "F.Cu") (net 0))
 (segment (start 139.08 97.28) (end 139.08 95) (width 0.25) (layer "F.Cu") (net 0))
 (segment (start 130.72 89.68) (end 130.72 79.04) (width 0.25) (layer "F.Cu") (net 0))
 (segment (start 144.4 91.2) (end 142.88 89.68) (width 0.25) (layer "F.Cu") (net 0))
 (segment (start 168.72 88.16) (end 168.72 82.08) (width 0.25) (layer "F.Cu") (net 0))
 (segment (start 143.3 69.92) (end 144.36 68.86) (width 0.25) (layer "F.Cu") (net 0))
 (segment (start 174.8 82.08) (end 171.76 79.04) (width 0.25) (layer "F.Cu") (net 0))
 (segment (start 142.88 71.44) (end 142.88 69.92) (width 0.25) (layer "F.Cu") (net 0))
 (segment (start 174.8 88.16) (end 174.8 82.08) (width 0.25) (layer "F.Cu") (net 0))
 (segment (start 171.76 74.48) (end 162.64 65.36) (width 0.25) (layer "F.Cu") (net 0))
 (segment (start 159.6 88.16) (end 159.6 86.64) (width 0.25) (layer "F.Cu") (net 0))
 (segment (start 142.88 89.68) (end 142.88 85.12) (width 0.25) (layer "F.Cu") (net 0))
 (segment (start 141.36 89.68) (end 141.36 84.56) (width 0.25) (layer "F.Cu") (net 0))
 (segment (start 166.44 97.28) (end 166.44 93.48) (width 0.25) (layer "F.Cu") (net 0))
 (segment (start 152.76 88.92) (end 153.52 88.16) (width 0.25) (layer "F.Cu") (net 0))
 (segment (start 161.88 97.28) (end 161.88 93.48) (width 0.25) (layer "F.Cu") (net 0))
 (segment (start 133.76 80.56) (end 142.88 71.44) (width 0.25) (layer "F.Cu") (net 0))
 (segment (start 141.36 84.56) (end 144.36 81.56) (width 0.25) (layer "F.Cu") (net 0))
 (segment (start 161.12 80.54) (end 159.6 79.02) (width 0.25) (layer "F.Cu") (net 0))
 (segment (start 142.88 77.52) (end 143.32 77.52) (width 0.25) (layer "F.Cu") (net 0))
 (segment (start 144.4 89.68) (end 144.36 89.64) (width 0.25) (layer "F.Cu") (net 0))
 (segment (start 161.12 85.12) (end 160.62 85.12) (width 0.25) (layer "F.Cu") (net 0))
 (segment (start 141.36 76) (end 141.36 74.4) (width 0.25) (layer "F.Cu") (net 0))
 (segment (start 139.84 69.92) (end 139.84 68.4) (width 0.25) (layer "F.Cu") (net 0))
 (segment (start 134.52 97.28) (end 134.52 95) (width 0.25) (layer "F.Cu") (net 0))
 (segment (start 167.2 82.08) (end 162.64 77.52) (width 0.25) (layer "F.Cu") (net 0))
 (segment (start 162.64 74.48) (end 162.64 71.44) (width 0.25) (layer "F.Cu") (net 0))
 (segment (start 164.16 74.48) (end 164.16 70.88) (width 0.25) (layer "F.Cu") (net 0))
 (segment (start 142.88 75.42) (end 144.36 73.94) (width 0.25) (layer "F.Cu") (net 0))
 (segment (start 170.24 82.08) (end 162.64 74.48) (width 0.25) (layer "F.Cu") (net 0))
 (segment (start 151.24 97.28) (end 151.24 88.92) (width 0.25) (layer "F.Cu") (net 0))
 (segment (start 143.64 97.28) (end 143.64 95) (width 0.25) (layer "F.Cu") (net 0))
 (segment (start 156.56 88.16) (end 157.06 87.66) (width 0.25) (layer "F.Cu") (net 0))
 (segment (start 145.16 95) (end 139.84 89.68) (width 0.25) (layer "F.Cu") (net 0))
 (segment (start 153.52 88.16) (end 156.56 88.16) (width 0.25) (layer "F.Cu") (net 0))
 (segment (start 165.68 74.48) (end 165.68 69.86) (width 0.25) (layer "F.Cu") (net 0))
 (segment (start 142.88 80.56) (end 142.88 80.5) (width 0.25) (layer "F.Cu") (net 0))
 (segment (start 168.72 82.08) (end 161.12 74.48) (width 0.25) (layer "F.Cu") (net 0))
 (segment (start 129.2 79.04) (end 138.32 69.92) (width 0.25) (layer "F.Cu") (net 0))
 (segment (start 147.44 91.2) (end 144.4 91.2) (width 0.25) (layer "F.Cu") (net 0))
 (segment (start 164.92 93.48) (end 170.24 88.16) (width 0.25) (layer "F.Cu") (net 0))
 (segment (start 149.72 97.28) (end 149.72 90.44) (width 0.25) (layer "F.Cu") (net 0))
 (segment (start 158.08 91.2) (end 161.12 88.16) (width 0.25) (layer "F.Cu") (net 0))
 (segment (start 139.84 83.6) (end 142.88 80.56) (width 0.25) (layer "F.Cu") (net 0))
 (segment (start 142.88 76) (end 142.88 75.42) (width 0.25) (layer "F.Cu") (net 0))
 (segment (start 161.12 88.16) (end 161.12 85.12) (width 0.25) (layer "F.Cu") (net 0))
 (segment (start 171.76 79.04) (end 171.76 74.48) (width 0.25) (layer "F.Cu") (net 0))
 (segment (start 161.12 72.92) (end 159.6 71.4) (width 0.25) (layer "F.Cu") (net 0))
 (segment (start 143.34 85.12) (end 144.36 84.1) (width 0.25) (layer "F.Cu") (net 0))
 (segment (start 171.76 82.08) (end 164.16 74.48) (width 0.25) (layer "F.Cu") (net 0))
 (segment (start 163.4 93.48) (end 168.72 88.16) (width 0.25) (layer "F.Cu") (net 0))
 (segment (start 160.36 93.48) (end 165.68 88.16) (width 0.25) (layer "F.Cu") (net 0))
 (segment (start 156.56 91.2) (end 158.08 91.2) (width 0.25) (layer "F.Cu") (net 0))
 (segment (start 142.88 80.5) (end 144.36 79.02) (width 0.25) (layer "F.Cu") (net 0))
 (segment (start 161.12 74.48) (end 161.12 72.92) (width 0.25) (layer "F.Cu") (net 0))
 (segment (start 169.48 97.28) (end 169.48 93.48) (width 0.25) (layer "F.Cu") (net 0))
 (segment (start 142.12 95) (end 136.8 89.68) (width 0.25) (layer "F.Cu") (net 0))
 (segment (start 139.84 68.4) (end 142.88 65.36) (width 0.25) (layer "F.Cu") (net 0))
 (segment (start 138.32 89.68) (end 138.32 83.6) (width 0.25) (layer "F.Cu") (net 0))
 (segment (start 162.18 71.44) (end 159.6 68.86) (width 0.25) (layer "F.Cu") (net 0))
 (segment (start 162.64 62.32) (end 161.56 61.24) (width 0.25) (layer "F.Cu") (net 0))
 (segment (start 161.56 61.24) (end 159.6 61.24) (width 0.25) (layer "F.Cu") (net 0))
 (segment (start 167.2 88.16) (end 167.2 82.08) (width 0.25) (layer "F.Cu") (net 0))
 (segment (start 141.36 71.44) (end 141.36 69.92) (width 0.25) (layer "F.Cu") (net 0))
 (segment (start 162.64 76.98) (end 159.6 73.94) (width 0.25) (layer "F.Cu") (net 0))
 (segment (start 142.12 97.28) (end 142.12 95) (width 0.25) (layer "F.Cu") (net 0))
 (segment (start 136.8 89.68) (end 136.8 83.6) (width 0.25) (layer "F.Cu") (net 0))
 (segment (start 161.12 80.56) (end 161.12 80.54) (width 0.25) (layer "F.Cu") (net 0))
 (segment (start 144.36 89.64) (end 144.36 86.64) (width 0.25) (layer "F.Cu") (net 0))
 (segment (start 142.88 85.12) (end 143.34 85.12) (width 0.25) (layer "F.Cu") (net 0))
 (segment (start 160.36 97.28) (end 160.36 93.48) (width 0.25) (layer "F.Cu") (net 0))
 (segment (start 139.84 89.68) (end 139.84 83.6) (width 0.25) (layer "F.Cu") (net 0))
 (segment (start 167.96 97.28) (end 167.96 93.48) (width 0.25) (layer "F.Cu") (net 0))
 (segment (start 143.64 95) (end 138.32 89.68) (width 0.25) (layer "F.Cu") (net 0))
 (segment (start 155.04 89.68) (end 158.08 89.68) (width 0.25) (layer "F.Cu") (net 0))
 (segment (start 160.62 85.12) (end 159.6 84.1) (width 0.25) (layer "F.Cu") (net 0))
 (segment (start 150.48 88.16) (end 147.44 88.16) (width 0.25) (layer "F.Cu") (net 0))
 (segment (start 136.04 95) (end 130.72 89.68) (width 0.25) (layer "F.Cu") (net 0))
 (segment (start 142.88 65.26) (end 144.36 63.78) (width 0.25) (layer "F.Cu") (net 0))
 (segment (start 151.24 88.92) (end 150.48 88.16) (width 0.25) (layer "F.Cu") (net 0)))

